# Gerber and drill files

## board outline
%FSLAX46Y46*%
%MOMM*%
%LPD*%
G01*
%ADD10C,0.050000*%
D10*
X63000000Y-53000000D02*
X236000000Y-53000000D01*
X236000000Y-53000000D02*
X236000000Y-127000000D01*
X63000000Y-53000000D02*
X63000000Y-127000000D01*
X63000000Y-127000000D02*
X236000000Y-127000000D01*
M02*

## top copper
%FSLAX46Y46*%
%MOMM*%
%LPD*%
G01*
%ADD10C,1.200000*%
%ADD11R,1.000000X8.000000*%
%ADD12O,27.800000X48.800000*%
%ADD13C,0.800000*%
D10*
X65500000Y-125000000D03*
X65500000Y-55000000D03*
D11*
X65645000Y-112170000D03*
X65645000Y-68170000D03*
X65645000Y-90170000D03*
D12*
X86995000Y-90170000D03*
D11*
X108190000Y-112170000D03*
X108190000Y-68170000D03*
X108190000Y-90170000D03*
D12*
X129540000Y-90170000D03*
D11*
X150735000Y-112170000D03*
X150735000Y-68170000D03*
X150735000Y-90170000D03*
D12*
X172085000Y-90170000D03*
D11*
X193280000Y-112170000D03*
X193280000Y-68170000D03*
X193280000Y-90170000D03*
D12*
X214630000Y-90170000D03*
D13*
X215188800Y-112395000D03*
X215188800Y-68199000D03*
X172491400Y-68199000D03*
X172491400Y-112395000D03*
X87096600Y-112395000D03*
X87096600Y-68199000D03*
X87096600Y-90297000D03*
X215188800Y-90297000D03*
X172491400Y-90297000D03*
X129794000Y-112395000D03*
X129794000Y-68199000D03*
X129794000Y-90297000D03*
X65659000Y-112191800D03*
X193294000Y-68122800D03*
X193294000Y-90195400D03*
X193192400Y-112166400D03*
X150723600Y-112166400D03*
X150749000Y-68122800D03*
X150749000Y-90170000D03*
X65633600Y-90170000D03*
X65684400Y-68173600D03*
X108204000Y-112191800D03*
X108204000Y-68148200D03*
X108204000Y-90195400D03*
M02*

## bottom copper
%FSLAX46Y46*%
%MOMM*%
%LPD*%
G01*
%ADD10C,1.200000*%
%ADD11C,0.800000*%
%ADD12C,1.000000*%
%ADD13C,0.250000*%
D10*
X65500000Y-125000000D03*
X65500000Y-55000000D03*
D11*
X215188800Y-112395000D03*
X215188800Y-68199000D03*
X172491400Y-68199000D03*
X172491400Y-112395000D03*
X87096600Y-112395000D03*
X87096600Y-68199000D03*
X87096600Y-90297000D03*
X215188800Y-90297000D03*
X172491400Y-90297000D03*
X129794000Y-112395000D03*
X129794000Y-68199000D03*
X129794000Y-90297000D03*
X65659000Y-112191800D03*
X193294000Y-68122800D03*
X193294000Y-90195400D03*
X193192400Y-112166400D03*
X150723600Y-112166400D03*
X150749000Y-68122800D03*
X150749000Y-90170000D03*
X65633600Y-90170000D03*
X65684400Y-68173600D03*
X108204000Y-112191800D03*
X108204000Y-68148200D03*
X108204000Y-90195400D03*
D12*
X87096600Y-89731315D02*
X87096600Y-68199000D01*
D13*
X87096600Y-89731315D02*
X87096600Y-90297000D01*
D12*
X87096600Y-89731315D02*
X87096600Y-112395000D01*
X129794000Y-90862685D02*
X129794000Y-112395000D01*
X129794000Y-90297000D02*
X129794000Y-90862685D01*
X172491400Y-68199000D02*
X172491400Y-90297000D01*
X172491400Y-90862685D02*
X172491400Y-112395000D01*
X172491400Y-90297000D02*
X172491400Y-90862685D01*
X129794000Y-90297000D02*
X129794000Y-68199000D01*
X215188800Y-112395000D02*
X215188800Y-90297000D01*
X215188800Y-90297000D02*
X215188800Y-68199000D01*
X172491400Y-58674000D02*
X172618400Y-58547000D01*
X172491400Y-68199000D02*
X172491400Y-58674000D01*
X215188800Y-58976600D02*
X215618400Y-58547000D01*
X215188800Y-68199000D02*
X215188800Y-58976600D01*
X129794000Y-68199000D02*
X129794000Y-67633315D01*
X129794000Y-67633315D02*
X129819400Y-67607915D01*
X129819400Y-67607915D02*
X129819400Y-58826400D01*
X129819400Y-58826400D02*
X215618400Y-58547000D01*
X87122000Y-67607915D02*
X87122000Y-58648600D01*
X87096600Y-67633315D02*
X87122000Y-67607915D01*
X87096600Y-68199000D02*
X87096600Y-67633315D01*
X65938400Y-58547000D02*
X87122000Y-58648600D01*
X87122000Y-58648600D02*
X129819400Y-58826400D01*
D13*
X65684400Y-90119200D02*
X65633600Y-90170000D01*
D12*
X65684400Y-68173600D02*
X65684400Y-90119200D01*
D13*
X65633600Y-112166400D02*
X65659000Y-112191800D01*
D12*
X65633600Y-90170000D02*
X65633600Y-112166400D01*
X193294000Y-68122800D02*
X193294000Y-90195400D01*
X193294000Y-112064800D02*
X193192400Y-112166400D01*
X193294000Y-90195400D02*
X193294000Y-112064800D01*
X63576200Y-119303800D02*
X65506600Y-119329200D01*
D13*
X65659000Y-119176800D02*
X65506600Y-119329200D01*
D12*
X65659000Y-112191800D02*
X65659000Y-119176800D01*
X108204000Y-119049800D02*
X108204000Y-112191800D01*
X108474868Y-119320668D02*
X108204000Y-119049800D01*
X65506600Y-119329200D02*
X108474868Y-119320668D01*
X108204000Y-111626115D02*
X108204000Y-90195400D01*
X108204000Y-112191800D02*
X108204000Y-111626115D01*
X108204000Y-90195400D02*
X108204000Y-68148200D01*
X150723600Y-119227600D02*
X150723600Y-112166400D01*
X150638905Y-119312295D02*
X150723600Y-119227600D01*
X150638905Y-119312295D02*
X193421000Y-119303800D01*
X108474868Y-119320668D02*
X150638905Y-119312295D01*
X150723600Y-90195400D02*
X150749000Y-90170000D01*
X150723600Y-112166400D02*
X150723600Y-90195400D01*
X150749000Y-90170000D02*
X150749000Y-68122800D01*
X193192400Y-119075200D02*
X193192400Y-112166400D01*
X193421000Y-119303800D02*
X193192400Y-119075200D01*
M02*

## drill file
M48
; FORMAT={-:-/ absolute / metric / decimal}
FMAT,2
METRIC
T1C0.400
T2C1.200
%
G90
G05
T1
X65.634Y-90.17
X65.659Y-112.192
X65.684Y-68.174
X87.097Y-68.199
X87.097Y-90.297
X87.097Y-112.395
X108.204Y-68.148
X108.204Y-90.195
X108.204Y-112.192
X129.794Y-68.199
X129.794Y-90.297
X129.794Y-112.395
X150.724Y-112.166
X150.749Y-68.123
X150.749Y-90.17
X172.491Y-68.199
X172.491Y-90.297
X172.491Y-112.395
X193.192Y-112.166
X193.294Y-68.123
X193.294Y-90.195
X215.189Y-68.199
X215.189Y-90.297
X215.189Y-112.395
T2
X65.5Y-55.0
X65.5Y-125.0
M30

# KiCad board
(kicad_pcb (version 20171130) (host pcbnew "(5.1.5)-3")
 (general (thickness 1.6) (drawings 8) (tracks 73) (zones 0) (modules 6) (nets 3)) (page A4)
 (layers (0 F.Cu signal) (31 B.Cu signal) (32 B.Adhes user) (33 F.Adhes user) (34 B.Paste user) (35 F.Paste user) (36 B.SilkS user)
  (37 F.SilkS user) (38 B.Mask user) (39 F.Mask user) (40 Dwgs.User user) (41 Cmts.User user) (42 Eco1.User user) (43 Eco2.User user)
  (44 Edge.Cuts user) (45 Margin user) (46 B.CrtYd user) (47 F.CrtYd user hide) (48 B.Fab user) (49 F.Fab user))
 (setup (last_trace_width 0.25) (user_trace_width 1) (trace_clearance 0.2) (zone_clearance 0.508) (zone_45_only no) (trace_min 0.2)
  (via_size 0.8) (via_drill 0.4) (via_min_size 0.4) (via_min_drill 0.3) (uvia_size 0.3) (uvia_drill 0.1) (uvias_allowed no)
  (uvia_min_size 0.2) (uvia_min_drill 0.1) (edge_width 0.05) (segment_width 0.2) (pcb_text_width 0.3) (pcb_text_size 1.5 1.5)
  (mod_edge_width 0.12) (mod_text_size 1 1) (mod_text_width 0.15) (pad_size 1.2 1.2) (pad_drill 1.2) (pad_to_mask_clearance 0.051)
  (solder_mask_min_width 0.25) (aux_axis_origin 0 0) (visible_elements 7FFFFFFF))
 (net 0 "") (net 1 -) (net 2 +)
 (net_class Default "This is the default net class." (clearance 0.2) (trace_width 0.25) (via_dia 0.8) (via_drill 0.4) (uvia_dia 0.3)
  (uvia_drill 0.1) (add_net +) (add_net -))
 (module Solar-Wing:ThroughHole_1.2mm (layer F.Cu) (at 65.5 125)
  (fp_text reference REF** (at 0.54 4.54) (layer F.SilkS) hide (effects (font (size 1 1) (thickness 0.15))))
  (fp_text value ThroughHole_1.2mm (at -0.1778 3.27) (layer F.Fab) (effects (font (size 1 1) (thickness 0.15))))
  (pad "" thru_hole circle (at 0 0) (size 1.2 1.2) (drill 1.2) (layers *.Cu *.Mask)))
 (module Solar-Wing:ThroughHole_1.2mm (layer F.Cu) (at 65.5 55)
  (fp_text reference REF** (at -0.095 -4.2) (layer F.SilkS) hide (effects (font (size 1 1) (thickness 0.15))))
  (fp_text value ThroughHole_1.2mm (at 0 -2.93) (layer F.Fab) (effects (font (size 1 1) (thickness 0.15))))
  (pad "" thru_hole circle (at 0 0) (size 1.2 1.2) (drill 1.2) (layers *.Cu *.Mask)))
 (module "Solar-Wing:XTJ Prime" (layer F.Cu) (at 86.995 90.17 90)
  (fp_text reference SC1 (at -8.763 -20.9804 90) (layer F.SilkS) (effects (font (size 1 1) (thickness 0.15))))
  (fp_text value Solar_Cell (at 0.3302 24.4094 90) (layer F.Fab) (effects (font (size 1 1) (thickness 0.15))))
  (pad 2 smd rect (at -22 -21.35 90) (size 8 1) (layers F.Cu F.Paste F.Mask) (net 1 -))
  (pad 2 smd rect (at 22 -21.35 90) (size 8 1) (layers F.Cu F.Paste F.Mask) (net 1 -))
  (pad 2 smd rect (at 0 -21.35 90) (size 8 1) (layers F.Cu F.Paste F.Mask) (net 1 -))
  (pad 1 smd oval (at 0 0 90) (size 48.8 27.8) (layers F.Cu F.Paste F.Mask) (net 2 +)))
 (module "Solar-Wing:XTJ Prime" (layer F.Cu) (at 129.54 90.17 90)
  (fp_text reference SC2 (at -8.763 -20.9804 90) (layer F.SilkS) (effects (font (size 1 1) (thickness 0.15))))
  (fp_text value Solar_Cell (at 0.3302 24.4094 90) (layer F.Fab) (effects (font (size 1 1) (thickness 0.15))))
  (pad 2 smd rect (at -22 -21.35 90) (size 8 1) (layers F.Cu F.Paste F.Mask) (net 1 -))
  (pad 2 smd rect (at 22 -21.35 90) (size 8 1) (layers F.Cu F.Paste F.Mask) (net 1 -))
  (pad 2 smd rect (at 0 -21.35 90) (size 8 1) (layers F.Cu F.Paste F.Mask) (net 1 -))
  (pad 1 smd oval (at 0 0 90) (size 48.8 27.8) (layers F.Cu F.Paste F.Mask) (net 2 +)))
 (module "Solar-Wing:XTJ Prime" (layer F.Cu) (at 172.085 90.17 90)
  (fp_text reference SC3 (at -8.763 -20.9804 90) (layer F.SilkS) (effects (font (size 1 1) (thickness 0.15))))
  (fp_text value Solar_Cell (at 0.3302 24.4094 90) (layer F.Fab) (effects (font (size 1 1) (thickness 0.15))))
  (pad 2 smd rect (at -22 -21.35 90) (size 8 1) (layers F.Cu F.Paste F.Mask) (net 1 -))
  (pad 2 smd rect (at 22 -21.35 90) (size 8 1) (layers F.Cu F.Paste F.Mask) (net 1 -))
  (pad 2 smd rect (at 0 -21.35 90) (size 8 1) (layers F.Cu F.Paste F.Mask) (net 1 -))
  (pad 1 smd oval (at 0 0 90) (size 48.8 27.8) (layers F.Cu F.Paste F.Mask) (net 2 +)))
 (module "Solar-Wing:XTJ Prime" (layer F.Cu) (at 214.63 90.17 90)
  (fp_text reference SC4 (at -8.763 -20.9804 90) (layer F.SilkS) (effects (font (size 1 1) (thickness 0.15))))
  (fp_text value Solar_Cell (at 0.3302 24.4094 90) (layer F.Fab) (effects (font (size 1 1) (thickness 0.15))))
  (pad 2 smd rect (at -22 -21.35 90) (size 8 1) (layers F.Cu F.Paste F.Mask) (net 1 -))
  (pad 2 smd rect (at 22 -21.35 90) (size 8 1) (layers F.Cu F.Paste F.Mask) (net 1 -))
  (pad 2 smd rect (at 0 -21.35 90) (size 8 1) (layers F.Cu F.Paste F.Mask) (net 1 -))
  (pad 1 smd oval (at 0 0 90) (size 48.8 27.8) (layers F.Cu F.Paste F.Mask) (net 2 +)))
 (gr_line (start 63 53) (end 236 53) (layer Edge.Cuts) (width 0.05))
 (gr_line (start 236 53) (end 236 127) (layer Edge.Cuts) (width 0.05))
 (gr_line (start 63 53) (end 63 127) (layer Edge.Cuts) (width 0.05))
 (gr_line (start 63 127) (end 236 127) (layer Edge.Cuts) (width 0.05))
 (via (at 215.1888 112.395) (size 0.8) (drill 0.4) (layers F.Cu B.Cu) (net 2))
 (via (at 215.1888 68.199) (size 0.8) (drill 0.4) (layers F.Cu B.Cu) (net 2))
 (via (at 172.4914 68.199) (size 0.8) (drill 0.4) (layers F.Cu B.Cu) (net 2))
 (via (at 172.4914 112.395) (size 0.8) (drill 0.4) (layers F.Cu B.Cu) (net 2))
 (via (at 87.0966 112.395) (size 0.8) (drill 0.4) (layers F.Cu B.Cu) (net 2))
 (via (at 87.0966 68.199) (size 0.8) (drill 0.4) (layers F.Cu B.Cu) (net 2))
 (via (at 87.0966 90.297) (size 0.8) (drill 0.4) (layers F.Cu B.Cu) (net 2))
 (via (at 215.1888 90.297) (size 0.8) (drill 0.4) (layers F.Cu B.Cu) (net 2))
 (via (at 172.4914 90.297) (size 0.8) (drill 0.4) (layers F.Cu B.Cu) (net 2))
 (via (at 129.794 112.395) (size 0.8) (drill 0.4) (layers F.Cu B.Cu) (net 2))
 (via (at 129.794 68.199) (size 0.8) (drill 0.4) (layers F.Cu B.Cu) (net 2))
 (via (at 129.794 90.297) (size 0.8) (drill 0.4) (layers F.Cu B.Cu) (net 2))
 (segment (start 87.0966 89.731315) (end 87.0966 68.199) (width 1) (layer B.Cu) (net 2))
 (segment (start 87.0966 89.731315) (end 87.0966 90.297) (width 0.25) (layer B.Cu) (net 2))
 (segment (start 87.0966 89.731315) (end 87.0966 112.395) (width 1) (layer B.Cu) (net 2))
 (segment (start 129.794 90.862685) (end 129.794 112.395) (width 1) (layer B.Cu) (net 2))
 (segment (start 129.794 90.297) (end 129.794 90.862685) (width 1) (layer B.Cu) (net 2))
 (segment (start 172.4914 68.199) (end 172.4914 90.297) (width 1) (layer B.Cu) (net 2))
 (segment (start 172.4914 90.862685) (end 172.4914 112.395) (width 1) (layer B.Cu) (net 2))
 (segment (start 172.4914 90.297) (end 172.4914 90.862685) (width 1) (layer B.Cu) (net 2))
 (segment (start 129.794 90.297) (end 129.794 68.199) (width 1) (layer B.Cu) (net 2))
 (segment (start 215.1888 112.395) (end 215.1888 90.297) (width 1) (layer B.Cu) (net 2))
 (segment (start 215.1888 90.297) (end 215.1888 68.199) (width 1) (layer B.Cu) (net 2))
 (segment (start 172.4914 58.674) (end 172.6184 58.547) (width 1) (layer B.Cu) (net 2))
 (segment (start 172.4914 68.199) (end 172.4914 58.674) (width 1) (layer B.Cu) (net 2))
 (segment (start 215.1888 58.9766) (end 215.6184 58.547) (width 1) (layer B.Cu) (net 2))
 (segment (start 215.1888 68.199) (end 215.1888 58.9766) (width 1) (layer B.Cu) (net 2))
 (segment (start 129.794 68.199) (end 129.794 67.633315) (width 1) (layer B.Cu) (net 2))
 (segment (start 129.794 67.633315) (end 129.8194 67.607915) (width 1) (layer B.Cu) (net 2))
 (segment (start 129.8194 67.607915) (end 129.8194 58.8264) (width 1) (layer B.Cu) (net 2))
 (segment (start 129.8194 58.8264) (end 215.6184 58.547) (width 1) (layer B.Cu) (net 2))
 (segment (start 87.122 67.607915) (end 87.122 58.6486) (width 1) (layer B.Cu) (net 2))
 (segment (start 87.0966 67.633315) (end 87.122 67.607915) (width 1) (layer B.Cu) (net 2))
 (segment (start 87.0966 68.199) (end 87.0966 67.633315) (width 1) (layer B.Cu) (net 2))
 (segment (start 65.9384 58.547) (end 87.122 58.6486) (width 1) (layer B.Cu) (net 2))
 (segment (start 87.122 58.6486) (end 129.8194 58.8264) (width 1) (layer B.Cu) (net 2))
 (via (at 65.659 112.1918) (size 0.8) (drill 0.4) (layers F.Cu B.Cu) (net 1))
 (via (at 193.294 68.1228) (size 0.8) (drill 0.4) (layers F.Cu B.Cu) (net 1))
 (via (at 193.294 90.1954) (size 0.8) (drill 0.4) (layers F.Cu B.Cu) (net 1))
 (via (at 193.1924 112.1664) (size 0.8) (drill 0.4) (layers F.Cu B.Cu) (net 1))
 (via (at 150.7236 112.1664) (size 0.8) (drill 0.4) (layers F.Cu B.Cu) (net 1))
 (via (at 150.749 68.1228) (size 0.8) (drill 0.4) (layers F.Cu B.Cu) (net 1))
 (via (at 150.749 90.17) (size 0.8) (drill 0.4) (layers F.Cu B.Cu) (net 1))
 (via (at 65.6336 90.17) (size 0.8) (drill 0.4) (layers F.Cu B.Cu) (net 1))
 (via (at 65.6844 68.1736) (size 0.8) (drill 0.4) (layers F.Cu B.Cu) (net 1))
 (via (at 108.204 112.1918) (size 0.8) (drill 0.4) (layers F.Cu B.Cu) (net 1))
 (via (at 108.204 68.1482) (size 0.8) (drill 0.4) (layers F.Cu B.Cu) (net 1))
 (via (at 108.204 90.1954) (size 0.8) (drill 0.4) (layers F.Cu B.Cu) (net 1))
 (segment (start 65.6844 90.1192) (end 65.6336 90.17) (width 0.25) (layer B.Cu) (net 1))
 (segment (start 65.6844 68.1736) (end 65.6844 90.1192) (width 1) (layer B.Cu) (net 1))
 (segment (start 65.6336 112.1664) (end 65.659 112.1918) (width 0.25) (layer B.Cu) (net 1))
 (segment (start 65.6336 90.17) (end 65.6336 112.1664) (width 1) (layer B.Cu) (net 1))
 (segment (start 193.294 68.1228) (end 193.294 90.1954) (width 1) (layer B.Cu) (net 1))
 (segment (start 193.294 112.0648) (end 193.1924 112.1664) (width 1) (layer B.Cu) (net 1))
 (segment (start 193.294 90.1954) (end 193.294 112.0648) (width 1) (layer B.Cu) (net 1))
 (segment (start 63.5762 119.3038) (end 65.5066 119.3292) (width 1) (layer B.Cu) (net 1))
 (segment (start 65.659 119.1768) (end 65.5066 119.3292) (width 0.25) (layer B.Cu) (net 1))
 (segment (start 65.659 112.1918) (end 65.659 119.1768) (width 1) (layer B.Cu) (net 1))
 (segment (start 108.204 119.0498) (end 108.204 112.1918) (width 1) (layer B.Cu) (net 1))
 (segment (start 108.474868 119.320668) (end 108.204 119.0498) (width 1) (layer B.Cu) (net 1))
 (segment (start 65.5066 119.3292) (end 108.474868 119.320668) (width 1) (layer B.Cu) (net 1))
 (segment (start 108.204 111.626115) (end 108.204 90.1954) (width 1) (layer B.Cu) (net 1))
 (segment (start 108.204 112.1918) (end 108.204 111.626115) (width 1) (layer B.Cu) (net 1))
 (segment (start 108.204 90.1954) (end 108.204 68.1482) (width 1) (layer B.Cu) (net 1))
 (segment (start 150.7236 119.2276) (end 150.7236 112.1664) (width 1) (layer B.Cu) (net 1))
 (segment (start 150.638905 119.312295) (end 150.7236 119.2276) (width 1) (layer B.Cu) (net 1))
 (segment (start 150.638905 119.312295) (end 193.421 119.3038) (width 1) (layer B.Cu) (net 1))
 (segment (start 108.474868 119.320668) (end 150.638905 119.312295) (width 1) (layer B.Cu) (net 1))
 (segment (start 150.7236 90.1954) (end 150.749 90.17) (width 1) (layer B.Cu) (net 1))
 (segment (start 150.7236 112.1664) (end 150.7236 90.1954) (width 1) (layer B.Cu) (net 1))
 (segment (start 150.749 90.17) (end 150.749 68.1228) (width 1) (layer B.Cu) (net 1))
 (segment (start 193.1924 119.0752) (end 193.1924 112.1664) (width 1) (layer B.Cu) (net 1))
 (segment (start 193.421 119.3038) (end 193.1924 119.0752) (width 1) (layer B.Cu) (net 1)))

